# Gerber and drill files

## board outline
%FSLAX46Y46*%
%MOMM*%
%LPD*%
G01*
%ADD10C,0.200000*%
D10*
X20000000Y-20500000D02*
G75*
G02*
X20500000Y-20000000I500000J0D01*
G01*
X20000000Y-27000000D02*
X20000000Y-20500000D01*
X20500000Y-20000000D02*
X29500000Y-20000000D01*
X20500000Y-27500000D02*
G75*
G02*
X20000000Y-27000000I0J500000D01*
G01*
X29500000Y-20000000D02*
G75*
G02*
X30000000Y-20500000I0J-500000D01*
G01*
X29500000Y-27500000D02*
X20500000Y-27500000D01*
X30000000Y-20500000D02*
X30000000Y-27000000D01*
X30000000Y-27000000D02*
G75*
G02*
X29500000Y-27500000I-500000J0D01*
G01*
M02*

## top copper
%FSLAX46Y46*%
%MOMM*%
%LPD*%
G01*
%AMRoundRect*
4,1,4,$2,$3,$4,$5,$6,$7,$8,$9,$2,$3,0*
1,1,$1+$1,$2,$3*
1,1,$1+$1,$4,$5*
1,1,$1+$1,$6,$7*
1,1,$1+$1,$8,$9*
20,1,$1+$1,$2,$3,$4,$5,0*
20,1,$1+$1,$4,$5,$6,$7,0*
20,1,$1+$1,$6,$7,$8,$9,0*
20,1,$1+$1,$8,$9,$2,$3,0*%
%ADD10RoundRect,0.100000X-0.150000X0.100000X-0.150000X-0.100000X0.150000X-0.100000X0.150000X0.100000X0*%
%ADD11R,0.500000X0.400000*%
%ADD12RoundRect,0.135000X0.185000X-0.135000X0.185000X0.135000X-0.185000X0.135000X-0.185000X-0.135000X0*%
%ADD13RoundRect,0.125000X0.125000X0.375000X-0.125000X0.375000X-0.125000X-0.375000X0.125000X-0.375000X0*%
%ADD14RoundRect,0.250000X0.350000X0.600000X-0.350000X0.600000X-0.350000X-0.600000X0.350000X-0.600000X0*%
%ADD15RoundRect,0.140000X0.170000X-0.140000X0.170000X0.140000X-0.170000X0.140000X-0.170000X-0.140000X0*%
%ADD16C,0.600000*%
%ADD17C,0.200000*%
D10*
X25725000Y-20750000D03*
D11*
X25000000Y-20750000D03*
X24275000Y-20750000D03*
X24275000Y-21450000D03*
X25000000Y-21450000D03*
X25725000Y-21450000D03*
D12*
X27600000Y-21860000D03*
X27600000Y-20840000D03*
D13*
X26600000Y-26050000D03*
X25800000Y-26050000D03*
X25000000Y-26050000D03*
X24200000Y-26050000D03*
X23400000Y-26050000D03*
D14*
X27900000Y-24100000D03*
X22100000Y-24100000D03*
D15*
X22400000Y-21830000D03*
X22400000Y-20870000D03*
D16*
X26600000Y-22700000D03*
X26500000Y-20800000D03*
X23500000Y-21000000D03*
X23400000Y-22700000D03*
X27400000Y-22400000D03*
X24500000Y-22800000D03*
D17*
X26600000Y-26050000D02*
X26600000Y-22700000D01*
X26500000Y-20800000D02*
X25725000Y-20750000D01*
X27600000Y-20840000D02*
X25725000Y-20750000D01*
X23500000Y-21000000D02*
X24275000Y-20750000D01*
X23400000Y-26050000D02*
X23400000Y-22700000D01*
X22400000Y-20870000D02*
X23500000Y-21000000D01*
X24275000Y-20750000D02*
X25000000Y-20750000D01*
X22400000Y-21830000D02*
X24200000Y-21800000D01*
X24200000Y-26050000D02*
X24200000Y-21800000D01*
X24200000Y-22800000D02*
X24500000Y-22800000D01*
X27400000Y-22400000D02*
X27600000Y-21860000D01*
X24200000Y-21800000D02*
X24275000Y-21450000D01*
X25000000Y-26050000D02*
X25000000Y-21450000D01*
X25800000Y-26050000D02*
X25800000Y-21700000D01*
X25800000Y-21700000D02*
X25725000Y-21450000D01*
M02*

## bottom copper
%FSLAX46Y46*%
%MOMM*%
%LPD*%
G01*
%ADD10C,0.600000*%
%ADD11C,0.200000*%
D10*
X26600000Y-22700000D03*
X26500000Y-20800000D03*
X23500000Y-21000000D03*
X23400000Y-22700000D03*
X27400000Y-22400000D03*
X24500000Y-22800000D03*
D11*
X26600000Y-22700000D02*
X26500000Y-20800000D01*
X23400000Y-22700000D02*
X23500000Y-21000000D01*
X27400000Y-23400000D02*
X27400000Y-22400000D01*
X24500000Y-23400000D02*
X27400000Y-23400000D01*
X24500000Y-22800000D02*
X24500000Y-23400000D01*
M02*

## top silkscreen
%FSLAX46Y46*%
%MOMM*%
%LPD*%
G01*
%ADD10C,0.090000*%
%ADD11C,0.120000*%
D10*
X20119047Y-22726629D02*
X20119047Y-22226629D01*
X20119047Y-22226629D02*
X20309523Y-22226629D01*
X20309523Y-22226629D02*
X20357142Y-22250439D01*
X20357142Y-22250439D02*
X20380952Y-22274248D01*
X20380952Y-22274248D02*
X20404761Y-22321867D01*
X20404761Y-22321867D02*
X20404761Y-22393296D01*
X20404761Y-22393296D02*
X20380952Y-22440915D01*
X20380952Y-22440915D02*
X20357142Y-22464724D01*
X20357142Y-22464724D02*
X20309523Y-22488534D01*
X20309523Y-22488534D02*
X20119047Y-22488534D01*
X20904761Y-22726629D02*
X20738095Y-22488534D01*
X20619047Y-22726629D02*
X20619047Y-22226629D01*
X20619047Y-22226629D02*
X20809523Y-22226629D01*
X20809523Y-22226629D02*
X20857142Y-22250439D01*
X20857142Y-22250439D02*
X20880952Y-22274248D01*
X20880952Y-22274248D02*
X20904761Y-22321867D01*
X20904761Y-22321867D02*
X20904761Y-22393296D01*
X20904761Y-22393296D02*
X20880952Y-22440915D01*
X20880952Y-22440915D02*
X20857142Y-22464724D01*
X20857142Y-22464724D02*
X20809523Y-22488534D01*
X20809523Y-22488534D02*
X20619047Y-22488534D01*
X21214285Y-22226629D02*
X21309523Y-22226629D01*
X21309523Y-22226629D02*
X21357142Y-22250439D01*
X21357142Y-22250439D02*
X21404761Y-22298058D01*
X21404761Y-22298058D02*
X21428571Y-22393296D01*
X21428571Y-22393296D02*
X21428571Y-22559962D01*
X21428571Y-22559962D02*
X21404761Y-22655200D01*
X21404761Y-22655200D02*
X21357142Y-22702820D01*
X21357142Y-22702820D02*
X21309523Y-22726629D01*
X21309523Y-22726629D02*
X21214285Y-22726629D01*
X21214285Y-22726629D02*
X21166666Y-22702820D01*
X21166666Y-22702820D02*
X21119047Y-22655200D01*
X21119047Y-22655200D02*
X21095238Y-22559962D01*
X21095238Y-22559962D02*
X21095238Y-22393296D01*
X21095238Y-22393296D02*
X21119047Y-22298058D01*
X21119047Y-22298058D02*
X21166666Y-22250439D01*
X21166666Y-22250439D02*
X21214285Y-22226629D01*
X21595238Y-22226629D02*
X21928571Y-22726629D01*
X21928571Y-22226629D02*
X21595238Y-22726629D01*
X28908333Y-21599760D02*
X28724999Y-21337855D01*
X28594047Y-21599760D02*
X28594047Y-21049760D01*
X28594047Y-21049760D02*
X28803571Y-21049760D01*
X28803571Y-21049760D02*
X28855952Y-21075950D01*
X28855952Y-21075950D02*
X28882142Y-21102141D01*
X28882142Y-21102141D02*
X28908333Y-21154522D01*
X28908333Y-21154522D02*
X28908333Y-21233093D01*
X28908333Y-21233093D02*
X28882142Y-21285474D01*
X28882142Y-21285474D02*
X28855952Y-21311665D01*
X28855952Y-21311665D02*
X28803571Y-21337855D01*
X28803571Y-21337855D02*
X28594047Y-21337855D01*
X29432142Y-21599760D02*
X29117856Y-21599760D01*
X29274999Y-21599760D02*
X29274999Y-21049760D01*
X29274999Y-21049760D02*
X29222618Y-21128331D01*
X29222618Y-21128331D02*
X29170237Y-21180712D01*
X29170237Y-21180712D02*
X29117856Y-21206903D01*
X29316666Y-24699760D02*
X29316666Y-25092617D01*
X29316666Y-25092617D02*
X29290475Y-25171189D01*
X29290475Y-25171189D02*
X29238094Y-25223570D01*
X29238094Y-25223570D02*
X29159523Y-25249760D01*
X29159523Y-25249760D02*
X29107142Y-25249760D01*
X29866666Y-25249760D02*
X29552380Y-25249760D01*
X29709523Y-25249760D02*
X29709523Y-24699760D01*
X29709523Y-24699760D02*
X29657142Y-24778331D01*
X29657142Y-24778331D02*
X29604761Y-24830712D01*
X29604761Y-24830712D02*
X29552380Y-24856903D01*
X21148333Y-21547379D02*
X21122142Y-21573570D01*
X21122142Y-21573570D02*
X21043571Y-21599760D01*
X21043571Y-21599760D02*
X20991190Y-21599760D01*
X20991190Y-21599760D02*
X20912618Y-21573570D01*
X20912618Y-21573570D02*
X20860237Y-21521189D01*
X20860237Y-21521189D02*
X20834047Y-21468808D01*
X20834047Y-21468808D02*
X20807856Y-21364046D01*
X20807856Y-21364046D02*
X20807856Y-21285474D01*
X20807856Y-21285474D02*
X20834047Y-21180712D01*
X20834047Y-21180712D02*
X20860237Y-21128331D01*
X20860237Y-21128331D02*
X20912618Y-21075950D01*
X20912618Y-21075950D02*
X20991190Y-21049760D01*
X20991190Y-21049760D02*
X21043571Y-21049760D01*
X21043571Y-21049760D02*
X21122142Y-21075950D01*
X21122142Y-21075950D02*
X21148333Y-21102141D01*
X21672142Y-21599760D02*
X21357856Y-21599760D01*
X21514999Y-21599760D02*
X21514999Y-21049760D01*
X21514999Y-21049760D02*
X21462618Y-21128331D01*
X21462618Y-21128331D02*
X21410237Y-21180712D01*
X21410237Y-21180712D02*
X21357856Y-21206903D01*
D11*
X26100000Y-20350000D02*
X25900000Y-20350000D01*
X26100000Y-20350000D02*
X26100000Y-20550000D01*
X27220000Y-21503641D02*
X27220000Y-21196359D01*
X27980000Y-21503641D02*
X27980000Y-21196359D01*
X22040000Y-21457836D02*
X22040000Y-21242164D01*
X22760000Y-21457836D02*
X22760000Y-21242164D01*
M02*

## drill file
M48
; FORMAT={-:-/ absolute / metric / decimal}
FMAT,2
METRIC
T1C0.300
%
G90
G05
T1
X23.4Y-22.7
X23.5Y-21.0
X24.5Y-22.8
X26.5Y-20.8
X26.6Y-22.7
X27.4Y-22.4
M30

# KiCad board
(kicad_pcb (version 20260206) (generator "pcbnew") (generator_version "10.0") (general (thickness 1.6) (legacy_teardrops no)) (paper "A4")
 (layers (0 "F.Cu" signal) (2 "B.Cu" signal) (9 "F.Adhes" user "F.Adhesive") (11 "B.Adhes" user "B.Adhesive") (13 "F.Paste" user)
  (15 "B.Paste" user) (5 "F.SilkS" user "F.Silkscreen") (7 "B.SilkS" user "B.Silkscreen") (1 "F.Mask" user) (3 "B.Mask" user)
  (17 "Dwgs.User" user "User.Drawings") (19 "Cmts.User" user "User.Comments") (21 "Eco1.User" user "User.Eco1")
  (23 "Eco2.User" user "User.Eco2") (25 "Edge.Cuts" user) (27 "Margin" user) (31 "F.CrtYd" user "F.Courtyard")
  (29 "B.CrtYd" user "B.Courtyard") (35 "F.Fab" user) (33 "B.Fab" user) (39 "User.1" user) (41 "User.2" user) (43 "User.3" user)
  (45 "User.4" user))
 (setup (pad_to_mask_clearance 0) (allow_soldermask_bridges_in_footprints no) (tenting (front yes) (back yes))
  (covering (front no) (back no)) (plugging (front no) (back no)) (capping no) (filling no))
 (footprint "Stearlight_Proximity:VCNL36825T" (layer "F.Cu") (at 25 21.1 -90)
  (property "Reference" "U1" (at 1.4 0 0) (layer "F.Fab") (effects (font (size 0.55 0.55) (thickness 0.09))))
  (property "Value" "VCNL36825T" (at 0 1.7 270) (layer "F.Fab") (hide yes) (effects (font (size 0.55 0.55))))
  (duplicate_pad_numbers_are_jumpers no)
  (fp_line (start -0.75 -1.1) (end -0.75 -0.9) (stroke (width 0.12) (type default)) (layer "F.SilkS"))
  (fp_line (start -0.75 -1.1) (end -0.55 -1.1) (stroke (width 0.12) (type default)) (layer "F.SilkS"))
  (pad "1" smd roundrect (at -0.35 -0.725 270) (size 0.4 0.5) (layers "F.Cu" "F.Mask" "F.Paste") (roundrect_rratio 0.25) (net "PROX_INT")
   (clearance 0.1) (thermal_bridge_angle 45))
  (pad "2" smd rect (at -0.35 0 270) (size 0.4 0.5) (layers "F.Cu" "F.Mask" "F.Paste") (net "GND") (clearance 0.1) (thermal_bridge_angle 45))
  (pad "3" smd rect (at -0.35 0.725 270) (size 0.4 0.5) (layers "F.Cu" "F.Mask" "F.Paste") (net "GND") (clearance 0.1)
   (thermal_bridge_angle 45))
  (pad "4" smd rect (at 0.35 0.725 270) (size 0.4 0.5) (layers "F.Cu" "F.Mask" "F.Paste") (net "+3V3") (clearance 0.1)
   (thermal_bridge_angle 45))
  (pad "5" smd rect (at 0.35 0 270) (size 0.4 0.5) (layers "F.Cu" "F.Mask" "F.Paste") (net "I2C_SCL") (clearance 0.1)
   (thermal_bridge_angle 45))
  (pad "6" smd rect (at 0.35 -0.725 270) (size 0.4 0.5) (layers "F.Cu" "F.Mask" "F.Paste") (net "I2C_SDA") (clearance 0.1)
   (thermal_bridge_angle 45)))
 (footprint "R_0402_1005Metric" (layer "F.Cu") (at 27.6 21.35 90)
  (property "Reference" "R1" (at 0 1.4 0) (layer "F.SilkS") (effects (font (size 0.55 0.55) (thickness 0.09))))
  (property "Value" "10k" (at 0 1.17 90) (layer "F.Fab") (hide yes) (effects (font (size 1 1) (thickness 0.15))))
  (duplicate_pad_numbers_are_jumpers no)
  (fp_line (start -0.153641 -0.38) (end 0.153641 -0.38) (stroke (width 0.12) (type solid)) (layer "F.SilkS"))
  (fp_line (start -0.153641 0.38) (end 0.153641 0.38) (stroke (width 0.12) (type solid)) (layer "F.SilkS"))
  (pad "1" smd roundrect (at -0.51 0 90) (size 0.54 0.64) (layers "F.Cu" "F.Mask" "F.Paste") (roundrect_rratio 0.25) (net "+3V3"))
  (pad "2" smd roundrect (at 0.51 0 90) (size 0.54 0.64) (layers "F.Cu" "F.Mask" "F.Paste") (roundrect_rratio 0.25) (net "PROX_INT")))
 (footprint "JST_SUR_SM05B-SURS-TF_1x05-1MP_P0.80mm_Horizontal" (layer "F.Cu") (at 25 24.9 180)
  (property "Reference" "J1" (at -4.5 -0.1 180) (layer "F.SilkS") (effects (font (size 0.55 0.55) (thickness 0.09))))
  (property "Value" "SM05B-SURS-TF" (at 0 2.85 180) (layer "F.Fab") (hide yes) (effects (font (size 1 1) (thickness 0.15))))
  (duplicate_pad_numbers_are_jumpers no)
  (pad "1" smd roundrect (at -1.6 -1.15 180) (size 0.5 1) (layers "F.Cu" "F.Mask" "F.Paste") (roundrect_rratio 0.25) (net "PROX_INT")
   (clearance 0.1))
  (pad "2" smd roundrect (at -0.8 -1.15 180) (size 0.5 1) (layers "F.Cu" "F.Mask" "F.Paste") (roundrect_rratio 0.25) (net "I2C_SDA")
   (clearance 0.1))
  (pad "3" smd roundrect (at 0 -1.15 180) (size 0.5 1) (layers "F.Cu" "F.Mask" "F.Paste") (roundrect_rratio 0.25) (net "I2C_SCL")
   (clearance 0.1))
  (pad "4" smd roundrect (at 0.8 -1.15 180) (size 0.5 1) (layers "F.Cu" "F.Mask" "F.Paste") (roundrect_rratio 0.25) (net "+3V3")
   (clearance 0.1))
  (pad "5" smd roundrect (at 1.6 -1.15 180) (size 0.5 1) (layers "F.Cu" "F.Mask" "F.Paste") (roundrect_rratio 0.25) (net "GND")
   (clearance 0.1))
  (pad "MP" smd roundrect (at -2.9 0.8 180) (size 1.2 1.7) (layers "F.Cu" "F.Mask" "F.Paste") (roundrect_rratio 0.208333) (clearance 0.1))
  (pad "MP" smd roundrect (at 2.9 0.8 180) (size 1.2 1.7) (layers "F.Cu" "F.Mask" "F.Paste") (roundrect_rratio 0.208333) (clearance 0.1)))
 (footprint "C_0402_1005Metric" (layer "F.Cu") (at 22.4 21.35 90)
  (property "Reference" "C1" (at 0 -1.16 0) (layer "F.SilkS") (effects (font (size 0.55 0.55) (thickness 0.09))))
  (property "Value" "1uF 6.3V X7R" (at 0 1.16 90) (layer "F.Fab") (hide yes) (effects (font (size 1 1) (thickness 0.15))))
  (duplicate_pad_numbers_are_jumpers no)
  (fp_line (start -0.107836 -0.36) (end 0.107836 -0.36) (stroke (width 0.12) (type solid)) (layer "F.SilkS"))
  (fp_line (start -0.107836 0.36) (end 0.107836 0.36) (stroke (width 0.12) (type solid)) (layer "F.SilkS"))
  (pad "1" smd roundrect (at -0.48 0 90) (size 0.56 0.62) (layers "F.Cu" "F.Mask" "F.Paste") (roundrect_rratio 0.25) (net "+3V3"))
  (pad "2" smd roundrect (at 0.48 0 90) (size 0.56 0.62) (layers "F.Cu" "F.Mask" "F.Paste") (roundrect_rratio 0.25) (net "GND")))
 (gr_arc (start 20 20.5) (mid 20.146447 20.146447) (end 20.5 20) (stroke (width 0.2) (type default)) (layer "Edge.Cuts"))
 (gr_line (start 20 27) (end 20 20.5) (stroke (width 0.2) (type default)) (layer "Edge.Cuts"))
 (gr_line (start 20.5 20) (end 29.5 20) (stroke (width 0.2) (type default)) (layer "Edge.Cuts"))
 (gr_arc (start 20.5 27.5) (mid 20.146447 27.353553) (end 20 27) (stroke (width 0.2) (type default)) (layer "Edge.Cuts"))
 (gr_arc (start 29.5 20) (mid 29.853553 20.146447) (end 30 20.5) (stroke (width 0.2) (type default)) (layer "Edge.Cuts"))
 (gr_line (start 29.5 27.5) (end 20.5 27.5) (stroke (width 0.2) (type default)) (layer "Edge.Cuts"))
 (gr_line (start 30 20.5) (end 30 27) (stroke (width 0.2) (type default)) (layer "Edge.Cuts"))
 (gr_arc (start 30 27) (mid 29.853553 27.353553) (end 29.5 27.5) (stroke (width 0.2) (type default)) (layer "Edge.Cuts"))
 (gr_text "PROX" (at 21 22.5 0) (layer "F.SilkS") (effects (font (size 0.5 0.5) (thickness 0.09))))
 (segment (start 26.6 26.05) (end 26.6 22.7) (width 0.2) (layer "F.Cu") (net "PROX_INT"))
 (segment (start 26.5 20.8) (end 25.725 20.75) (width 0.2) (layer "F.Cu") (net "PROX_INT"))
 (segment (start 27.6 20.84) (end 25.725 20.75) (width 0.2) (layer "F.Cu") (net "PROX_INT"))
 (via (at 26.6 22.7) (size 0.6) (drill 0.3) (layers "F.Cu" "B.Cu") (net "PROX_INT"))
 (via (at 26.5 20.8) (size 0.6) (drill 0.3) (layers "F.Cu" "B.Cu") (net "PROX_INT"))
 (segment (start 26.6 22.7) (end 26.5 20.8) (width 0.2) (layer "B.Cu") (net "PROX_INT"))
 (segment (start 23.5 21) (end 24.275 20.75) (width 0.2) (layer "F.Cu") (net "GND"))
 (segment (start 23.4 26.05) (end 23.4 22.7) (width 0.2) (layer "F.Cu") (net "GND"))
 (segment (start 22.4 20.87) (end 23.5 21) (width 0.2) (layer "F.Cu") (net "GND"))
 (segment (start 24.275 20.75) (end 25 20.75) (width 0.2) (layer "F.Cu") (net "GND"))
 (via (at 23.5 21) (size 0.6) (drill 0.3) (layers "F.Cu" "B.Cu") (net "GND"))
 (via (at 23.4 22.7) (size 0.6) (drill 0.3) (layers "F.Cu" "B.Cu") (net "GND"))
 (segment (start 23.4 22.7) (end 23.5 21) (width 0.2) (layer "B.Cu") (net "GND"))
 (segment (start 22.4 21.83) (end 24.2 21.8) (width 0.2) (layer "F.Cu") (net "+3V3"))
 (segment (start 24.2 26.05) (end 24.2 21.8) (width 0.2) (layer "F.Cu") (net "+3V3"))
 (segment (start 24.2 22.8) (end 24.5 22.8) (width 0.2) (layer "F.Cu") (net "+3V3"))
 (segment (start 27.4 22.4) (end 27.6 21.86) (width 0.2) (layer "F.Cu") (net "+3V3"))
 (segment (start 24.2 21.8) (end 24.275 21.45) (width 0.2) (layer "F.Cu") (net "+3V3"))
 (via (at 27.4 22.4) (size 0.6) (drill 0.3) (layers "F.Cu" "B.Cu") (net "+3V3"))
 (via (at 24.5 22.8) (size 0.6) (drill 0.3) (layers "F.Cu" "B.Cu") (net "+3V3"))
 (segment (start 27.4 23.4) (end 27.4 22.4) (width 0.2) (layer "B.Cu") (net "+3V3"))
 (segment (start 24.5 23.4) (end 27.4 23.4) (width 0.2) (layer "B.Cu") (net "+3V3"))
 (segment (start 24.5 22.8) (end 24.5 23.4) (width 0.2) (layer "B.Cu") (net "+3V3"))
 (segment (start 25 26.05) (end 25 21.45) (width 0.2) (layer "F.Cu") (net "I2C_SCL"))
 (segment (start 25.8 26.05) (end 25.8 21.7) (width 0.2) (layer "F.Cu") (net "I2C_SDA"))
 (segment (start 25.8 21.7) (end 25.725 21.45) (width 0.2) (layer "F.Cu") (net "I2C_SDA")))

